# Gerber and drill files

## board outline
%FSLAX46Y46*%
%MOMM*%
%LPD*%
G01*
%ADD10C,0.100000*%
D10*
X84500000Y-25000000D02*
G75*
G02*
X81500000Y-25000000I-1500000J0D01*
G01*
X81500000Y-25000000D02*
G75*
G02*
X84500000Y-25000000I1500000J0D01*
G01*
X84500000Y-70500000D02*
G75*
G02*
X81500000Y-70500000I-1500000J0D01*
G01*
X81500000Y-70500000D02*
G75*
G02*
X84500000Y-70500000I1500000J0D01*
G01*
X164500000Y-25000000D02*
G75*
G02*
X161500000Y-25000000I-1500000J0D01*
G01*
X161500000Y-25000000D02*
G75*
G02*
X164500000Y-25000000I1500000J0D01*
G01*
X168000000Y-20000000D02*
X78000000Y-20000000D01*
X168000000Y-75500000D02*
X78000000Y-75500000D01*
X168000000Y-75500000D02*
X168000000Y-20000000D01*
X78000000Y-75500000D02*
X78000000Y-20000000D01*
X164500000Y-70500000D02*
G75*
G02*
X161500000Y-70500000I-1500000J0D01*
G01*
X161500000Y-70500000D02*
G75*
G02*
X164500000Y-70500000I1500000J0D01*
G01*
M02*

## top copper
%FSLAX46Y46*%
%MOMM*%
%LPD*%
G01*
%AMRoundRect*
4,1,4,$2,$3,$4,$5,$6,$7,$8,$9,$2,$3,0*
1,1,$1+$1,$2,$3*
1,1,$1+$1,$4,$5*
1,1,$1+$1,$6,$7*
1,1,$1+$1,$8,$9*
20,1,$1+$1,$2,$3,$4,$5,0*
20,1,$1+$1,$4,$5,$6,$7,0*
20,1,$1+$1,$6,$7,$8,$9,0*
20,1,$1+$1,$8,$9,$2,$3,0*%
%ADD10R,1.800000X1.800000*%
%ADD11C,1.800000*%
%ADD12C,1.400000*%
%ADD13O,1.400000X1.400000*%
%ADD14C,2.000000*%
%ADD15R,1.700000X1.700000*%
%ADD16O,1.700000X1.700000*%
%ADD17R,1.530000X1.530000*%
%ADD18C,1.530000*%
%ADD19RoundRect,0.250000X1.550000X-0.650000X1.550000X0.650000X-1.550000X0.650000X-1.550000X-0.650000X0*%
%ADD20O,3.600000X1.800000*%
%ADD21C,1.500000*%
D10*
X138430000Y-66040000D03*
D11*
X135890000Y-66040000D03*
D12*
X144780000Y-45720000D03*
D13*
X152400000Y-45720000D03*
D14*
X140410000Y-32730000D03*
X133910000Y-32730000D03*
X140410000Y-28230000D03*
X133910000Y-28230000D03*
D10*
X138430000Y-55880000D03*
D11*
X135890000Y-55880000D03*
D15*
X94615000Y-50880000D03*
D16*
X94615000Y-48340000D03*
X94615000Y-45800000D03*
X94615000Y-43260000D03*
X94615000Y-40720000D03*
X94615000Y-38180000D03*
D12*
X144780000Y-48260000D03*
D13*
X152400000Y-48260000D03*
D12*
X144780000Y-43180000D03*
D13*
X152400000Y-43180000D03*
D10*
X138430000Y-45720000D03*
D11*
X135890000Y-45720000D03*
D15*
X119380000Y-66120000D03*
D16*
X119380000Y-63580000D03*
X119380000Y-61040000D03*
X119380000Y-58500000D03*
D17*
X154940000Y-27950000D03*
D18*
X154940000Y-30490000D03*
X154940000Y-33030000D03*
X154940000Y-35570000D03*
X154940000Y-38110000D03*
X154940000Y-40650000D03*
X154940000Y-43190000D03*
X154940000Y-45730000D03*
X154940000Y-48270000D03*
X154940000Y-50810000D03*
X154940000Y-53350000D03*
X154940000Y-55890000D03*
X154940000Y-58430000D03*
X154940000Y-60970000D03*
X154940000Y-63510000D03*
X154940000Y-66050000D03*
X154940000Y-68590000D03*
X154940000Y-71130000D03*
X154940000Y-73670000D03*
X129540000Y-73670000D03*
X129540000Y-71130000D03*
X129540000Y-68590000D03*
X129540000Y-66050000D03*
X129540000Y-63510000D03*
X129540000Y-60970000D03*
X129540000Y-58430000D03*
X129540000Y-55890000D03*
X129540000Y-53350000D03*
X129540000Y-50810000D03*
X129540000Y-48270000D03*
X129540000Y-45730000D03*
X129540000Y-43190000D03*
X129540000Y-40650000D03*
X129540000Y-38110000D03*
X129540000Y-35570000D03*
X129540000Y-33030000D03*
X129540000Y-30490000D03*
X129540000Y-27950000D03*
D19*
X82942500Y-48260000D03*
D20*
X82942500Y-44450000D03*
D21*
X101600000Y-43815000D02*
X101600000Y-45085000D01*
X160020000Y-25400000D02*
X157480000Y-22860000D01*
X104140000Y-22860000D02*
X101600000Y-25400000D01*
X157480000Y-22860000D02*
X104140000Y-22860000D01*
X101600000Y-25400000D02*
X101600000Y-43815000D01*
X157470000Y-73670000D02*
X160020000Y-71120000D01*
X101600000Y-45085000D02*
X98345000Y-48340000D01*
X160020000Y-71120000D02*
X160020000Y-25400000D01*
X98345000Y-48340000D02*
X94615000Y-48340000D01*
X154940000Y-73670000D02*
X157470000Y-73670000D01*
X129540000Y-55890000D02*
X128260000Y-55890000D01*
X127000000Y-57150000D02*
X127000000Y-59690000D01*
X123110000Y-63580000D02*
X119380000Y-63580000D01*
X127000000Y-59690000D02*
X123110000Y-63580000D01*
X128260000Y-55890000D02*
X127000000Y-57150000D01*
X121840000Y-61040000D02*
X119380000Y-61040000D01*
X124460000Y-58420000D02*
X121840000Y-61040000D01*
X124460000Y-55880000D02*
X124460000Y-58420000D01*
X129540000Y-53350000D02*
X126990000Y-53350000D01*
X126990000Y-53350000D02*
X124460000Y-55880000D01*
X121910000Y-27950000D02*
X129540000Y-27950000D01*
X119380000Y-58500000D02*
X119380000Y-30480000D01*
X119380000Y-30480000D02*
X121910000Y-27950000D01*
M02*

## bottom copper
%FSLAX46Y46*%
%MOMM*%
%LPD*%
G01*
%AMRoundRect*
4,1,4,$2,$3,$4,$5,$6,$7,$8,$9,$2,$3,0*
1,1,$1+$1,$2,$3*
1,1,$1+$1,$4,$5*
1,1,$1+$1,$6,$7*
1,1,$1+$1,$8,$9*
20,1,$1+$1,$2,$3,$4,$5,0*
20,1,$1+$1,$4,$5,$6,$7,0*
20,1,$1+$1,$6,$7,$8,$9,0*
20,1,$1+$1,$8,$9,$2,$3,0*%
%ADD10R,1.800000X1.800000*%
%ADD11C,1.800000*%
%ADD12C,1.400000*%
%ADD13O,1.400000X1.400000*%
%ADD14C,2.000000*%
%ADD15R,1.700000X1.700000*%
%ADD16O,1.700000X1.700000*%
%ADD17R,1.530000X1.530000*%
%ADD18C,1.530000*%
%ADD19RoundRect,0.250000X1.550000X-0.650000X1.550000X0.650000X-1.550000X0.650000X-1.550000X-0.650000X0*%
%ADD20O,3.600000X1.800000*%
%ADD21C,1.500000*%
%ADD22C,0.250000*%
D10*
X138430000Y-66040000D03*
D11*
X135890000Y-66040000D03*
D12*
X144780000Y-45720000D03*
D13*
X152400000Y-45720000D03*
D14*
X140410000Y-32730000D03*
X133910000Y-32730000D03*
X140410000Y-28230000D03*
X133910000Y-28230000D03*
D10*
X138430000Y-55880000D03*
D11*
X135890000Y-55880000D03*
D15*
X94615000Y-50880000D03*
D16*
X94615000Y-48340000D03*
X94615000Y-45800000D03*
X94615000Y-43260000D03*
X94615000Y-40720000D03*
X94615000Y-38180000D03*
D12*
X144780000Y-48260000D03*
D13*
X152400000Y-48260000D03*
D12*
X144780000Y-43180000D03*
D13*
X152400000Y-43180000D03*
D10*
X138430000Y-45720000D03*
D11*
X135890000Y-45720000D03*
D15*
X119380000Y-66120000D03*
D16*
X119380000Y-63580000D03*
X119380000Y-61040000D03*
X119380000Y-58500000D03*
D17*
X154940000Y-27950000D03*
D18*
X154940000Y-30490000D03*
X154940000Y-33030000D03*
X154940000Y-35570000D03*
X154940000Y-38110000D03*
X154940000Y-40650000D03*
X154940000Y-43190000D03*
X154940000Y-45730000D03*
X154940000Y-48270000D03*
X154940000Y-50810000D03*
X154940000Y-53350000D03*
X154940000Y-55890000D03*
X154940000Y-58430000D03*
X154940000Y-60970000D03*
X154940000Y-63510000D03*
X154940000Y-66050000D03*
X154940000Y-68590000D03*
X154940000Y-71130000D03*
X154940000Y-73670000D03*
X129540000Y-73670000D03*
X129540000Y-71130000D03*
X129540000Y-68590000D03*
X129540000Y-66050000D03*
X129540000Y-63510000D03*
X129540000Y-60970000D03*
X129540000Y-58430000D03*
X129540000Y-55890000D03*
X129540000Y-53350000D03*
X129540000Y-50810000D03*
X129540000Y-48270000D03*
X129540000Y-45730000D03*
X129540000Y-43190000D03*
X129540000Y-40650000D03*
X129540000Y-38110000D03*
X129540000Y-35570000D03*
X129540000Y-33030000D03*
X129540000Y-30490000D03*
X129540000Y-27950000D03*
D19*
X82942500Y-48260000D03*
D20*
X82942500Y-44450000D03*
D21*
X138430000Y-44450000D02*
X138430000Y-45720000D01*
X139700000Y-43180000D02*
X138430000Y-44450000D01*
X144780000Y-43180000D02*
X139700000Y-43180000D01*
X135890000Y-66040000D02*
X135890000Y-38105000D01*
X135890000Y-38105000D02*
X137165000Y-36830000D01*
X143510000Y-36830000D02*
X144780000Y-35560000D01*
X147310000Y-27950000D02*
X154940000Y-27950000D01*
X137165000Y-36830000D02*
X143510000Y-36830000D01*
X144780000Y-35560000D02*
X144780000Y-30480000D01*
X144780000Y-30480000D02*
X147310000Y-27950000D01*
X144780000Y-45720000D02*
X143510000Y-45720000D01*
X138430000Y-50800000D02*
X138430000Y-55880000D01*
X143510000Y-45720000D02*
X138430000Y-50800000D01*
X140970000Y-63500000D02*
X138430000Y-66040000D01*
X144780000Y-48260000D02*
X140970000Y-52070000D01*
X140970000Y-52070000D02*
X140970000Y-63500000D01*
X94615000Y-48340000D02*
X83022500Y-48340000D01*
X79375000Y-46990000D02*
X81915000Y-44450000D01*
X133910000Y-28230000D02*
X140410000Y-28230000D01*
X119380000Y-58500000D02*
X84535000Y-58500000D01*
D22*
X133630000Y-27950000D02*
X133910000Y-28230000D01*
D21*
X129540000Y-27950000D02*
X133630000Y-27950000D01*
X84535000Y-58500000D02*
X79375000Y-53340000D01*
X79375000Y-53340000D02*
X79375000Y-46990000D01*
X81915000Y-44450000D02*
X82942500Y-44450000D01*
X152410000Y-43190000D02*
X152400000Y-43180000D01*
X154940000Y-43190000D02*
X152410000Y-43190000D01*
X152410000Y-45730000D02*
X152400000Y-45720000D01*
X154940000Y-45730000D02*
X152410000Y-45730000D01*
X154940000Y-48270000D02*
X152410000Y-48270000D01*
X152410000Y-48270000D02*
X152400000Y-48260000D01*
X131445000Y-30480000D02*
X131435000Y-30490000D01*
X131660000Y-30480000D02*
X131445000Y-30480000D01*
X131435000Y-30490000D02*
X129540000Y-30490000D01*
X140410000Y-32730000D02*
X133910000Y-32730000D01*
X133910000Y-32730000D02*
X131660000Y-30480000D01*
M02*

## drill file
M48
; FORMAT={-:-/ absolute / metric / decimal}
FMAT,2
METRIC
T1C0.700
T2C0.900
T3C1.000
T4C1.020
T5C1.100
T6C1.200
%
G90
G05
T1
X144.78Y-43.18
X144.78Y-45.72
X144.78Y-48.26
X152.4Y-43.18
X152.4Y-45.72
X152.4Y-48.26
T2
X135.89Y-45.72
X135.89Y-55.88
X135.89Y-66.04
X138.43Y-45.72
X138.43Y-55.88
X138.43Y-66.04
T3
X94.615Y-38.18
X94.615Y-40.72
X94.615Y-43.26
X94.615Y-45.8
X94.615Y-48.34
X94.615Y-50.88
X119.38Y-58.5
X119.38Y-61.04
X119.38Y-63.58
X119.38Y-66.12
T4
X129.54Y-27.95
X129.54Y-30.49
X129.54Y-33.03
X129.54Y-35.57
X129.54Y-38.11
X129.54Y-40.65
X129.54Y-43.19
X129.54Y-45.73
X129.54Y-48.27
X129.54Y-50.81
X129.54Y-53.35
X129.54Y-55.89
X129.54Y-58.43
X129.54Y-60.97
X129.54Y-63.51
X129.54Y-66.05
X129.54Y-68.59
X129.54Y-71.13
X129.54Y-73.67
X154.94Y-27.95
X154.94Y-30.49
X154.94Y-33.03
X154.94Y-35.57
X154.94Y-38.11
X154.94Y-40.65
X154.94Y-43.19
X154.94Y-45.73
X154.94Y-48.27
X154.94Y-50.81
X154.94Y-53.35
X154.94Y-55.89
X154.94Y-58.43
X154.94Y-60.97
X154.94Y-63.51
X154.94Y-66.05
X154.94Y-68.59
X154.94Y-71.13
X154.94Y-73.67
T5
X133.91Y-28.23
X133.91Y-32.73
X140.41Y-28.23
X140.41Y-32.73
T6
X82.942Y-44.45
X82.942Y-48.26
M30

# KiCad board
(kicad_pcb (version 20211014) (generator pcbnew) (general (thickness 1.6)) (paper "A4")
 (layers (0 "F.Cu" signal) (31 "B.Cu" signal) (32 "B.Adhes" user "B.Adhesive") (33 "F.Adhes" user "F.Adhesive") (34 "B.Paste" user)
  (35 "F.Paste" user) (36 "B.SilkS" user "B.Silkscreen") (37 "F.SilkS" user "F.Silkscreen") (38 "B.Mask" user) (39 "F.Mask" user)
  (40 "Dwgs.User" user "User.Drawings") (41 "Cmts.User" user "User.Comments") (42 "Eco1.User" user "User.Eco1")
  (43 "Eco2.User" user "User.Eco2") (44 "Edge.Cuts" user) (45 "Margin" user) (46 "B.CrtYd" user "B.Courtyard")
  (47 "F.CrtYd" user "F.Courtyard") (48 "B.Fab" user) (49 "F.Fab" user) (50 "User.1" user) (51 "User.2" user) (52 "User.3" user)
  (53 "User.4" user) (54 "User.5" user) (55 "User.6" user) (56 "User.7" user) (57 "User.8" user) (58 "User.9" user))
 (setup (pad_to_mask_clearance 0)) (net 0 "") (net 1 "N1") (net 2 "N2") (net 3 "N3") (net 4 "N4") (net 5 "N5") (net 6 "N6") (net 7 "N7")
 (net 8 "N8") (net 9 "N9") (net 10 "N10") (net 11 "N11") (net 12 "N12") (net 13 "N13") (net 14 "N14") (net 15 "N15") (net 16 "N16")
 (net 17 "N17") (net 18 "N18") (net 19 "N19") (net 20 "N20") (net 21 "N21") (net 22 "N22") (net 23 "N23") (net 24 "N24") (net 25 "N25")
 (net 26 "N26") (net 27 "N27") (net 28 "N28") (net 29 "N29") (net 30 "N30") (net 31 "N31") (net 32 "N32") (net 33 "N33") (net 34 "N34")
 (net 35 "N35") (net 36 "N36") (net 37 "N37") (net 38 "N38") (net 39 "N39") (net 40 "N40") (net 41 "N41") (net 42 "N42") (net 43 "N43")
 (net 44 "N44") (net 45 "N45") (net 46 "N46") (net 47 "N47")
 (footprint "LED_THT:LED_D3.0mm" (layer "F.Cu") (at 138.43 66.04 180)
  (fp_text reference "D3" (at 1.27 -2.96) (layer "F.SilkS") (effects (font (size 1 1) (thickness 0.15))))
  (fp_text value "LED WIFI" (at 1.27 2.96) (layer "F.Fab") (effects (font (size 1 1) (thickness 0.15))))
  (pad "1" thru_hole rect (at 0 0 180) (size 1.8 1.8) (drill 0.9) (layers *.Cu *.Mask) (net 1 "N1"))
  (pad "2" thru_hole circle (at 2.54 0 180) (size 1.8 1.8) (drill 0.9) (layers *.Cu *.Mask) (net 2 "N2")))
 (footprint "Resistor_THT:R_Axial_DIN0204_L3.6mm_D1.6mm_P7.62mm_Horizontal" (layer "F.Cu") (at 144.78 45.72)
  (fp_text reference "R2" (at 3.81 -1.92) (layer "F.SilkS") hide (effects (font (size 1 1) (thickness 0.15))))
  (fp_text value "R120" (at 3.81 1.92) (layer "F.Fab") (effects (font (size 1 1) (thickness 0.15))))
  (pad "1" thru_hole circle (at 0 0) (size 1.4 1.4) (drill 0.7) (layers *.Cu *.Mask) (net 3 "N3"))
  (pad "2" thru_hole oval (at 7.62 0) (size 1.4 1.4) (drill 0.7) (layers *.Cu *.Mask) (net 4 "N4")))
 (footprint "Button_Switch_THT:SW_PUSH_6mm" (layer "F.Cu") (at 140.41 32.73 180)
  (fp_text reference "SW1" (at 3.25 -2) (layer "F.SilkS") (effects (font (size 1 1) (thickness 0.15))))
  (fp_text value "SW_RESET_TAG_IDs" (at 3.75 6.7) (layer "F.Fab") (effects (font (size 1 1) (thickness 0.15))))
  (pad "1" thru_hole circle (at 0 0 270) (size 2 2) (drill 1.1) (layers *.Cu *.Mask) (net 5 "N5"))
  (pad "1" thru_hole circle (at 6.5 0 270) (size 2 2) (drill 1.1) (layers *.Cu *.Mask) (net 5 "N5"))
  (pad "2" thru_hole circle (at 0 4.5 270) (size 2 2) (drill 1.1) (layers *.Cu *.Mask) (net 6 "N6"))
  (pad "2" thru_hole circle (at 6.5 4.5 270) (size 2 2) (drill 1.1) (layers *.Cu *.Mask) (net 6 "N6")))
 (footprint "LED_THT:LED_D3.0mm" (layer "F.Cu") (at 138.43 55.88 180)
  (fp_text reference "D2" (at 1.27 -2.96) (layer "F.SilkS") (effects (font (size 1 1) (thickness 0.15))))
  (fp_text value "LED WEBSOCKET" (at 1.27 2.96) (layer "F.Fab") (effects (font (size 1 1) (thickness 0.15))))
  (pad "1" thru_hole rect (at 0 0 180) (size 1.8 1.8) (drill 0.9) (layers *.Cu *.Mask) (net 3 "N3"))
  (pad "2" thru_hole circle (at 2.54 0 180) (size 1.8 1.8) (drill 0.9) (layers *.Cu *.Mask) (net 2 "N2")))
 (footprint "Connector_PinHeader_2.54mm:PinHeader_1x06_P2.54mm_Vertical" (layer "F.Cu") (at 94.615 50.88 180)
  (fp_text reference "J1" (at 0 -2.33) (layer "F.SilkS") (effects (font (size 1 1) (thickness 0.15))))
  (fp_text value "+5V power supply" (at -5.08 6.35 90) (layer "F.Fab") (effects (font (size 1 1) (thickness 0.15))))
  (pad "1" thru_hole rect (at 0 0 180) (size 1.7 1.7) (drill 1) (layers *.Cu *.Mask) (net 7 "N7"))
  (pad "2" thru_hole oval (at 0 2.54 180) (size 1.7 1.7) (drill 1) (layers *.Cu *.Mask) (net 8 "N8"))
  (pad "3" thru_hole oval (at 0 5.08 180) (size 1.7 1.7) (drill 1) (layers *.Cu *.Mask) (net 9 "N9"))
  (pad "4" thru_hole oval (at 0 7.62 180) (size 1.7 1.7) (drill 1) (layers *.Cu *.Mask) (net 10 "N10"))
  (pad "5" thru_hole oval (at 0 10.16 180) (size 1.7 1.7) (drill 1) (layers *.Cu *.Mask) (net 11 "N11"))
  (pad "6" thru_hole oval (at 0 12.7 180) (size 1.7 1.7) (drill 1) (layers *.Cu *.Mask) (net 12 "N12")))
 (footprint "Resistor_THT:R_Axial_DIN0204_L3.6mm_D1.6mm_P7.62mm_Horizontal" (layer "F.Cu") (at 144.78 48.26)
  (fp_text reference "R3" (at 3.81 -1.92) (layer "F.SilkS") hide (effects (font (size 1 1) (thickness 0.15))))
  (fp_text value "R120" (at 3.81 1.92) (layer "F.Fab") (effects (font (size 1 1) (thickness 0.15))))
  (pad "1" thru_hole circle (at 0 0) (size 1.4 1.4) (drill 0.7) (layers *.Cu *.Mask) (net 1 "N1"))
  (pad "2" thru_hole oval (at 7.62 0) (size 1.4 1.4) (drill 0.7) (layers *.Cu *.Mask) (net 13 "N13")))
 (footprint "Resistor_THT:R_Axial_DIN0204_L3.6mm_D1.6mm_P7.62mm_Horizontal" (layer "F.Cu") (at 144.78 43.18)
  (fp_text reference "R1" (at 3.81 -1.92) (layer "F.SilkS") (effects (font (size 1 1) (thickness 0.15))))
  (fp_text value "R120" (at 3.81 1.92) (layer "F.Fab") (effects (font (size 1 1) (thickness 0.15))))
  (pad "1" thru_hole circle (at 0 0) (size 1.4 1.4) (drill 0.7) (layers *.Cu *.Mask) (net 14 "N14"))
  (pad "2" thru_hole oval (at 7.62 0) (size 1.4 1.4) (drill 0.7) (layers *.Cu *.Mask) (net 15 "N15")))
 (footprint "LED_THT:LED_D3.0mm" (layer "F.Cu") (at 138.43 45.72 180)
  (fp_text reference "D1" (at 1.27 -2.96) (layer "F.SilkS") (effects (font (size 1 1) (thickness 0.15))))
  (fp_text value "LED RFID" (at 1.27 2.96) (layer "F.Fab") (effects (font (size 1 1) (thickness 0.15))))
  (pad "1" thru_hole rect (at 0 0 180) (size 1.8 1.8) (drill 0.9) (layers *.Cu *.Mask) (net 14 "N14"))
  (pad "2" thru_hole circle (at 2.54 0 180) (size 1.8 1.8) (drill 0.9) (layers *.Cu *.Mask) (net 2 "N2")))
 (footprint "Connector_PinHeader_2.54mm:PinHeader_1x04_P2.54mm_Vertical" (layer "F.Cu") (at 119.38 66.12 180)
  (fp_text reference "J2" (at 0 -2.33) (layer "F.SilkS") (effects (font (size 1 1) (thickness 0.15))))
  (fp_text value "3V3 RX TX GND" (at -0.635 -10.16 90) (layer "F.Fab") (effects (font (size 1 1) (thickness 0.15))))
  (pad "1" thru_hole rect (at 0 0 180) (size 1.7 1.7) (drill 1) (layers *.Cu *.Mask) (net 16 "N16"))
  (pad "2" thru_hole oval (at 0 2.54 180) (size 1.7 1.7) (drill 1) (layers *.Cu *.Mask) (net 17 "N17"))
  (pad "3" thru_hole oval (at 0 5.08 180) (size 1.7 1.7) (drill 1) (layers *.Cu *.Mask) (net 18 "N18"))
  (pad "4" thru_hole oval (at 0 7.62 180) (size 1.7 1.7) (drill 1) (layers *.Cu *.Mask) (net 6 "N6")))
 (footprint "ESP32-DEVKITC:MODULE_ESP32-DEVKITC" (layer "B.Cu") (at 142.24 50.8 180)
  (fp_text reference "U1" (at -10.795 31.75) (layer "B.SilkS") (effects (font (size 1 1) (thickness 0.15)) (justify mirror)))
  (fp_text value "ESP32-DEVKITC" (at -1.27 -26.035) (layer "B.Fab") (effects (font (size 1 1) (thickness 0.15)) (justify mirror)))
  (pad "1" thru_hole rect locked (at -12.7 22.85 180) (size 1.53 1.53) (drill 1.02) (layers *.Cu *.Mask) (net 2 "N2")
   (solder_mask_margin 0.102))
  (pad "2" thru_hole circle locked (at -12.7 20.31 180) (size 1.53 1.53) (drill 1.02) (layers *.Cu *.Mask) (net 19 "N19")
   (solder_mask_margin 0.102))
  (pad "3" thru_hole circle locked (at -12.7 17.77 180) (size 1.53 1.53) (drill 1.02) (layers *.Cu *.Mask) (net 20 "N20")
   (solder_mask_margin 0.102))
  (pad "4" thru_hole circle locked (at -12.7 15.23 180) (size 1.53 1.53) (drill 1.02) (layers *.Cu *.Mask) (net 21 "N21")
   (solder_mask_margin 0.102))
  (pad "5" thru_hole circle locked (at -12.7 12.69 180) (size 1.53 1.53) (drill 1.02) (layers *.Cu *.Mask) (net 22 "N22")
   (solder_mask_margin 0.102))
  (pad "6" thru_hole circle locked (at -12.7 10.15 180) (size 1.53 1.53) (drill 1.02) (layers *.Cu *.Mask) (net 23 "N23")
   (solder_mask_margin 0.102))
  (pad "7" thru_hole circle locked (at -12.7 7.61 180) (size 1.53 1.53) (drill 1.02) (layers *.Cu *.Mask) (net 15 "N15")
   (solder_mask_margin 0.102))
  (pad "8" thru_hole circle locked (at -12.7 5.07 180) (size 1.53 1.53) (drill 1.02) (layers *.Cu *.Mask) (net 4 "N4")
   (solder_mask_margin 0.102))
  (pad "9" thru_hole circle locked (at -12.7 2.53 180) (size 1.53 1.53) (drill 1.02) (layers *.Cu *.Mask) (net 13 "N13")
   (solder_mask_margin 0.102))
  (pad "10" thru_hole circle locked (at -12.7 -0.01 180) (size 1.53 1.53) (drill 1.02) (layers *.Cu *.Mask) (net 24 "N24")
   (solder_mask_margin 0.102))
  (pad "11" thru_hole circle locked (at -12.7 -2.55 180) (size 1.53 1.53) (drill 1.02) (layers *.Cu *.Mask) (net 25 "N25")
   (solder_mask_margin 0.102))
  (pad "12" thru_hole circle locked (at -12.7 -5.09 180) (size 1.53 1.53) (drill 1.02) (layers *.Cu *.Mask) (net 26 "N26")
   (solder_mask_margin 0.102))
  (pad "13" thru_hole circle locked (at -12.7 -7.63 180) (size 1.53 1.53) (drill 1.02) (layers *.Cu *.Mask) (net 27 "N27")
   (solder_mask_margin 0.102))
  (pad "14" thru_hole circle locked (at -12.7 -10.17 180) (size 1.53 1.53) (drill 1.02) (layers *.Cu *.Mask) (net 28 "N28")
   (solder_mask_margin 0.102))
  (pad "15" thru_hole circle locked (at -12.7 -12.71 180) (size 1.53 1.53) (drill 1.02) (layers *.Cu *.Mask) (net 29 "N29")
   (solder_mask_margin 0.102))
  (pad "16" thru_hole circle locked (at -12.7 -15.25 180) (size 1.53 1.53) (drill 1.02) (layers *.Cu *.Mask) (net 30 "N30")
   (solder_mask_margin 0.102))
  (pad "17" thru_hole circle locked (at -12.7 -17.79 180) (size 1.53 1.53) (drill 1.02) (layers *.Cu *.Mask) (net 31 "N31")
   (solder_mask_margin 0.102))
  (pad "18" thru_hole circle locked (at -12.7 -20.33 180) (size 1.53 1.53) (drill 1.02) (layers *.Cu *.Mask) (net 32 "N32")
   (solder_mask_margin 0.102))
  (pad "19" thru_hole circle locked (at -12.7 -22.87 180) (size 1.53 1.53) (drill 1.02) (layers *.Cu *.Mask) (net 8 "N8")
   (solder_mask_margin 0.102))
  (pad "20" thru_hole circle locked (at 12.7 -22.87 180) (size 1.53 1.53) (drill 1.02) (layers *.Cu *.Mask) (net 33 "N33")
   (solder_mask_margin 0.102))
  (pad "21" thru_hole circle locked (at 12.7 -20.33 180) (size 1.53 1.53) (drill 1.02) (layers *.Cu *.Mask) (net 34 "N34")
   (solder_mask_margin 0.102))
  (pad "22" thru_hole circle locked (at 12.7 -17.79 180) (size 1.53 1.53) (drill 1.02) (layers *.Cu *.Mask) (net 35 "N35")
   (solder_mask_margin 0.102))
  (pad "23" thru_hole circle locked (at 12.7 -15.25 180) (size 1.53 1.53) (drill 1.02) (layers *.Cu *.Mask) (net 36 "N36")
   (solder_mask_margin 0.102))
  (pad "24" thru_hole circle locked (at 12.7 -12.71 180) (size 1.53 1.53) (drill 1.02) (layers *.Cu *.Mask) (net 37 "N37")
   (solder_mask_margin 0.102))
  (pad "25" thru_hole circle locked (at 12.7 -10.17 180) (size 1.53 1.53) (drill 1.02) (layers *.Cu *.Mask) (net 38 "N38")
   (solder_mask_margin 0.102))
  (pad "26" thru_hole circle locked (at 12.7 -7.63 180) (size 1.53 1.53) (drill 1.02) (layers *.Cu *.Mask) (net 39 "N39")
   (solder_mask_margin 0.102))
  (pad "27" thru_hole circle locked (at 12.7 -5.09 180) (size 1.53 1.53) (drill 1.02) (layers *.Cu *.Mask) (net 17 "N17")
   (solder_mask_margin 0.102))
  (pad "28" thru_hole circle locked (at 12.7 -2.55 180) (size 1.53 1.53) (drill 1.02) (layers *.Cu *.Mask) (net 18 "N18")
   (solder_mask_margin 0.102))
  (pad "29" thru_hole circle locked (at 12.7 -0.01 180) (size 1.53 1.53) (drill 1.02) (layers *.Cu *.Mask) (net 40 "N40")
   (solder_mask_margin 0.102))
  (pad "30" thru_hole circle locked (at 12.7 2.53 180) (size 1.53 1.53) (drill 1.02) (layers *.Cu *.Mask) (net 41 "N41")
   (solder_mask_margin 0.102))
  (pad "31" thru_hole circle locked (at 12.7 5.07 180) (size 1.53 1.53) (drill 1.02) (layers *.Cu *.Mask) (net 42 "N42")
   (solder_mask_margin 0.102))
  (pad "32" thru_hole circle locked (at 12.7 7.61 180) (size 1.53 1.53) (drill 1.02) (layers *.Cu *.Mask) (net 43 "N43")
   (solder_mask_margin 0.102))
  (pad "33" thru_hole circle locked (at 12.7 10.15 180) (size 1.53 1.53) (drill 1.02) (layers *.Cu *.Mask) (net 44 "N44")
   (solder_mask_margin 0.102))
  (pad "34" thru_hole circle locked (at 12.7 12.69 180) (size 1.53 1.53) (drill 1.02) (layers *.Cu *.Mask) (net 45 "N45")
   (solder_mask_margin 0.102))
  (pad "35" thru_hole circle locked (at 12.7 15.23 180) (size 1.53 1.53) (drill 1.02) (layers *.Cu *.Mask) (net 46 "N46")
   (solder_mask_margin 0.102))
  (pad "36" thru_hole circle locked (at 12.7 17.77 180) (size 1.53 1.53) (drill 1.02) (layers *.Cu *.Mask) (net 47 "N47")
   (solder_mask_margin 0.102))
  (pad "37" thru_hole circle locked (at 12.7 20.31 180) (size 1.53 1.53) (drill 1.02) (layers *.Cu *.Mask) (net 5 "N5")
   (solder_mask_margin 0.102))
  (pad "38" thru_hole circle locked (at 12.7 22.85 180) (size 1.53 1.53) (drill 1.02) (layers *.Cu *.Mask) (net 6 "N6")
   (solder_mask_margin 0.102)))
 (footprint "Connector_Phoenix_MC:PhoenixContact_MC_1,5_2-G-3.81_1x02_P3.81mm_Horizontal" (layer "B.Cu") (at 82.9425 48.26 90)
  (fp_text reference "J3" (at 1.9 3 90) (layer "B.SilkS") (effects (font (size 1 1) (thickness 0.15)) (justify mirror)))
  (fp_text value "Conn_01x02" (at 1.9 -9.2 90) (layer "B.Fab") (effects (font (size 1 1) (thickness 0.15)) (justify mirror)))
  (pad "1" thru_hole roundrect (at 0 0 90) (size 1.8 3.6) (drill 1.2) (layers *.Cu *.Mask) (roundrect_rratio 0.138889) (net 8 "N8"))
  (pad "2" thru_hole oval (at 3.81 0 90) (size 1.8 3.6) (drill 1.2) (layers *.Cu *.Mask) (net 6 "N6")))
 (gr_circle (center 83 25) (end 84.5 25) (layer "Edge.Cuts") (width 0.1) (fill none))
 (gr_circle (center 83 70.5) (end 84.5 70.5) (layer "Edge.Cuts") (width 0.1) (fill none))
 (gr_circle (center 163 25) (end 164.5 25) (layer "Edge.Cuts") (width 0.1) (fill none))
 (gr_line (start 168 20) (end 78 20) (layer "Edge.Cuts") (width 0.1))
 (gr_line (start 168 75.5) (end 78 75.5) (layer "Edge.Cuts") (width 0.1))
 (gr_line (start 168 75.5) (end 168 20) (layer "Edge.Cuts") (width 0.1))
 (gr_line (start 78 75.5) (end 78 20) (layer "Edge.Cuts") (width 0.1))
 (gr_circle (center 163 70.5) (end 164.5 70.5) (layer "Edge.Cuts") (width 0.1) (fill none))
 (segment (start 138.43 44.45) (end 138.43 45.72) (width 1.5) (layer "B.Cu") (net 14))
 (segment (start 139.7 43.18) (end 138.43 44.45) (width 1.5) (layer "B.Cu") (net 14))
 (segment (start 144.78 43.18) (end 139.7 43.18) (width 1.5) (layer "B.Cu") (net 14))
 (segment (start 135.89 66.04) (end 135.89 38.105) (width 1.5) (layer "B.Cu") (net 2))
 (segment (start 135.89 38.105) (end 137.165 36.83) (width 1.5) (layer "B.Cu") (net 2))
 (segment (start 143.51 36.83) (end 144.78 35.56) (width 1.5) (layer "B.Cu") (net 2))
 (segment (start 147.31 27.95) (end 154.94 27.95) (width 1.5) (layer "B.Cu") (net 2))
 (segment (start 137.165 36.83) (end 143.51 36.83) (width 1.5) (layer "B.Cu") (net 2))
 (segment (start 144.78 35.56) (end 144.78 30.48) (width 1.5) (layer "B.Cu") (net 2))
 (segment (start 144.78 30.48) (end 147.31 27.95) (width 1.5) (layer "B.Cu") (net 2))
 (segment (start 144.78 45.72) (end 143.51 45.72) (width 1.5) (layer "B.Cu") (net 3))
 (segment (start 138.43 50.8) (end 138.43 55.88) (width 1.5) (layer "B.Cu") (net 3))
 (segment (start 143.51 45.72) (end 138.43 50.8) (width 1.5) (layer "B.Cu") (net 3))
 (segment (start 140.97 63.5) (end 138.43 66.04) (width 1.5) (layer "B.Cu") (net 1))
 (segment (start 144.78 48.26) (end 140.97 52.07) (width 1.5) (layer "B.Cu") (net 1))
 (segment (start 140.97 52.07) (end 140.97 63.5) (width 1.5) (layer "B.Cu") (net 1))
 (segment (start 101.6 43.815) (end 101.6 45.085) (width 1.5) (layer "F.Cu") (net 8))
 (segment (start 160.02 25.4) (end 157.48 22.86) (width 1.5) (layer "F.Cu") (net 8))
 (segment (start 104.14 22.86) (end 101.6 25.4) (width 1.5) (layer "F.Cu") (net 8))
 (segment (start 157.48 22.86) (end 104.14 22.86) (width 1.5) (layer "F.Cu") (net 8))
 (segment (start 101.6 25.4) (end 101.6 43.815) (width 1.5) (layer "F.Cu") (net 8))
 (segment (start 157.47 73.67) (end 160.02 71.12) (width 1.5) (layer "F.Cu") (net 8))
 (segment (start 101.6 45.085) (end 98.345 48.34) (width 1.5) (layer "F.Cu") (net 8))
 (segment (start 160.02 71.12) (end 160.02 25.4) (width 1.5) (layer "F.Cu") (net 8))
 (segment (start 98.345 48.34) (end 94.615 48.34) (width 1.5) (layer "F.Cu") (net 8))
 (segment (start 154.94 73.67) (end 157.47 73.67) (width 1.5) (layer "F.Cu") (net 8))
 (segment (start 94.615 48.34) (end 83.0225 48.34) (width 1.5) (layer "B.Cu") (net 8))
 (segment (start 129.54 55.89) (end 128.26 55.89) (width 1.5) (layer "F.Cu") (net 17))
 (segment (start 127 57.15) (end 127 59.69) (width 1.5) (layer "F.Cu") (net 17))
 (segment (start 123.11 63.58) (end 119.38 63.58) (width 1.5) (layer "F.Cu") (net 17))
 (segment (start 127 59.69) (end 123.11 63.58) (width 1.5) (layer "F.Cu") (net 17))
 (segment (start 128.26 55.89) (end 127 57.15) (width 1.5) (layer "F.Cu") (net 17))
 (segment (start 121.84 61.04) (end 119.38 61.04) (width 1.5) (layer "F.Cu") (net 18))
 (segment (start 124.46 58.42) (end 121.84 61.04) (width 1.5) (layer "F.Cu") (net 18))
 (segment (start 124.46 55.88) (end 124.46 58.42) (width 1.5) (layer "F.Cu") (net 18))
 (segment (start 129.54 53.35) (end 126.99 53.35) (width 1.5) (layer "F.Cu") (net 18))
 (segment (start 126.99 53.35) (end 124.46 55.88) (width 1.5) (layer "F.Cu") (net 18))
 (segment (start 121.91 27.95) (end 129.54 27.95) (width 1.5) (layer "F.Cu") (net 6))
 (segment (start 119.38 58.5) (end 119.38 30.48) (width 1.5) (layer "F.Cu") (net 6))
 (segment (start 119.38 30.48) (end 121.91 27.95) (width 1.5) (layer "F.Cu") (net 6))
 (segment (start 79.375 46.99) (end 81.915 44.45) (width 1.5) (layer "B.Cu") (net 6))
 (segment (start 133.91 28.23) (end 140.41 28.23) (width 1.5) (layer "B.Cu") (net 6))
 (segment (start 119.38 58.5) (end 84.535 58.5) (width 1.5) (layer "B.Cu") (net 6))
 (segment (start 133.63 27.95) (end 133.91 28.23) (width 0.25) (layer "B.Cu") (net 6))
 (segment (start 129.54 27.95) (end 133.63 27.95) (width 1.5) (layer "B.Cu") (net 6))
 (segment (start 84.535 58.5) (end 79.375 53.34) (width 1.5) (layer "B.Cu") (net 6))
 (segment (start 79.375 53.34) (end 79.375 46.99) (width 1.5) (layer "B.Cu") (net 6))
 (segment (start 81.915 44.45) (end 82.9425 44.45) (width 1.5) (layer "B.Cu") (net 6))
 (segment (start 152.41 43.19) (end 152.4 43.18) (width 1.5) (layer "B.Cu") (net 15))
 (segment (start 154.94 43.19) (end 152.41 43.19) (width 1.5) (layer "B.Cu") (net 15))
 (segment (start 152.41 45.73) (end 152.4 45.72) (width 1.5) (layer "B.Cu") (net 4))
 (segment (start 154.94 45.73) (end 152.41 45.73) (width 1.5) (layer "B.Cu") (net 4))
 (segment (start 154.94 48.27) (end 152.41 48.27) (width 1.5) (layer "B.Cu") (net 13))
 (segment (start 152.41 48.27) (end 152.4 48.26) (width 1.5) (layer "B.Cu") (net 13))
 (segment (start 131.445 30.48) (end 131.435 30.49) (width 1.5) (layer "B.Cu") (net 5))
 (segment (start 131.66 30.48) (end 131.445 30.48) (width 1.5) (layer "B.Cu") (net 5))
 (segment (start 131.435 30.49) (end 129.54 30.49) (width 1.5) (layer "B.Cu") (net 5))
 (segment (start 140.41 32.73) (end 133.91 32.73) (width 1.5) (layer "B.Cu") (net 5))
 (segment (start 133.91 32.73) (end 131.66 30.48) (width 1.5) (layer "B.Cu") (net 5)))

